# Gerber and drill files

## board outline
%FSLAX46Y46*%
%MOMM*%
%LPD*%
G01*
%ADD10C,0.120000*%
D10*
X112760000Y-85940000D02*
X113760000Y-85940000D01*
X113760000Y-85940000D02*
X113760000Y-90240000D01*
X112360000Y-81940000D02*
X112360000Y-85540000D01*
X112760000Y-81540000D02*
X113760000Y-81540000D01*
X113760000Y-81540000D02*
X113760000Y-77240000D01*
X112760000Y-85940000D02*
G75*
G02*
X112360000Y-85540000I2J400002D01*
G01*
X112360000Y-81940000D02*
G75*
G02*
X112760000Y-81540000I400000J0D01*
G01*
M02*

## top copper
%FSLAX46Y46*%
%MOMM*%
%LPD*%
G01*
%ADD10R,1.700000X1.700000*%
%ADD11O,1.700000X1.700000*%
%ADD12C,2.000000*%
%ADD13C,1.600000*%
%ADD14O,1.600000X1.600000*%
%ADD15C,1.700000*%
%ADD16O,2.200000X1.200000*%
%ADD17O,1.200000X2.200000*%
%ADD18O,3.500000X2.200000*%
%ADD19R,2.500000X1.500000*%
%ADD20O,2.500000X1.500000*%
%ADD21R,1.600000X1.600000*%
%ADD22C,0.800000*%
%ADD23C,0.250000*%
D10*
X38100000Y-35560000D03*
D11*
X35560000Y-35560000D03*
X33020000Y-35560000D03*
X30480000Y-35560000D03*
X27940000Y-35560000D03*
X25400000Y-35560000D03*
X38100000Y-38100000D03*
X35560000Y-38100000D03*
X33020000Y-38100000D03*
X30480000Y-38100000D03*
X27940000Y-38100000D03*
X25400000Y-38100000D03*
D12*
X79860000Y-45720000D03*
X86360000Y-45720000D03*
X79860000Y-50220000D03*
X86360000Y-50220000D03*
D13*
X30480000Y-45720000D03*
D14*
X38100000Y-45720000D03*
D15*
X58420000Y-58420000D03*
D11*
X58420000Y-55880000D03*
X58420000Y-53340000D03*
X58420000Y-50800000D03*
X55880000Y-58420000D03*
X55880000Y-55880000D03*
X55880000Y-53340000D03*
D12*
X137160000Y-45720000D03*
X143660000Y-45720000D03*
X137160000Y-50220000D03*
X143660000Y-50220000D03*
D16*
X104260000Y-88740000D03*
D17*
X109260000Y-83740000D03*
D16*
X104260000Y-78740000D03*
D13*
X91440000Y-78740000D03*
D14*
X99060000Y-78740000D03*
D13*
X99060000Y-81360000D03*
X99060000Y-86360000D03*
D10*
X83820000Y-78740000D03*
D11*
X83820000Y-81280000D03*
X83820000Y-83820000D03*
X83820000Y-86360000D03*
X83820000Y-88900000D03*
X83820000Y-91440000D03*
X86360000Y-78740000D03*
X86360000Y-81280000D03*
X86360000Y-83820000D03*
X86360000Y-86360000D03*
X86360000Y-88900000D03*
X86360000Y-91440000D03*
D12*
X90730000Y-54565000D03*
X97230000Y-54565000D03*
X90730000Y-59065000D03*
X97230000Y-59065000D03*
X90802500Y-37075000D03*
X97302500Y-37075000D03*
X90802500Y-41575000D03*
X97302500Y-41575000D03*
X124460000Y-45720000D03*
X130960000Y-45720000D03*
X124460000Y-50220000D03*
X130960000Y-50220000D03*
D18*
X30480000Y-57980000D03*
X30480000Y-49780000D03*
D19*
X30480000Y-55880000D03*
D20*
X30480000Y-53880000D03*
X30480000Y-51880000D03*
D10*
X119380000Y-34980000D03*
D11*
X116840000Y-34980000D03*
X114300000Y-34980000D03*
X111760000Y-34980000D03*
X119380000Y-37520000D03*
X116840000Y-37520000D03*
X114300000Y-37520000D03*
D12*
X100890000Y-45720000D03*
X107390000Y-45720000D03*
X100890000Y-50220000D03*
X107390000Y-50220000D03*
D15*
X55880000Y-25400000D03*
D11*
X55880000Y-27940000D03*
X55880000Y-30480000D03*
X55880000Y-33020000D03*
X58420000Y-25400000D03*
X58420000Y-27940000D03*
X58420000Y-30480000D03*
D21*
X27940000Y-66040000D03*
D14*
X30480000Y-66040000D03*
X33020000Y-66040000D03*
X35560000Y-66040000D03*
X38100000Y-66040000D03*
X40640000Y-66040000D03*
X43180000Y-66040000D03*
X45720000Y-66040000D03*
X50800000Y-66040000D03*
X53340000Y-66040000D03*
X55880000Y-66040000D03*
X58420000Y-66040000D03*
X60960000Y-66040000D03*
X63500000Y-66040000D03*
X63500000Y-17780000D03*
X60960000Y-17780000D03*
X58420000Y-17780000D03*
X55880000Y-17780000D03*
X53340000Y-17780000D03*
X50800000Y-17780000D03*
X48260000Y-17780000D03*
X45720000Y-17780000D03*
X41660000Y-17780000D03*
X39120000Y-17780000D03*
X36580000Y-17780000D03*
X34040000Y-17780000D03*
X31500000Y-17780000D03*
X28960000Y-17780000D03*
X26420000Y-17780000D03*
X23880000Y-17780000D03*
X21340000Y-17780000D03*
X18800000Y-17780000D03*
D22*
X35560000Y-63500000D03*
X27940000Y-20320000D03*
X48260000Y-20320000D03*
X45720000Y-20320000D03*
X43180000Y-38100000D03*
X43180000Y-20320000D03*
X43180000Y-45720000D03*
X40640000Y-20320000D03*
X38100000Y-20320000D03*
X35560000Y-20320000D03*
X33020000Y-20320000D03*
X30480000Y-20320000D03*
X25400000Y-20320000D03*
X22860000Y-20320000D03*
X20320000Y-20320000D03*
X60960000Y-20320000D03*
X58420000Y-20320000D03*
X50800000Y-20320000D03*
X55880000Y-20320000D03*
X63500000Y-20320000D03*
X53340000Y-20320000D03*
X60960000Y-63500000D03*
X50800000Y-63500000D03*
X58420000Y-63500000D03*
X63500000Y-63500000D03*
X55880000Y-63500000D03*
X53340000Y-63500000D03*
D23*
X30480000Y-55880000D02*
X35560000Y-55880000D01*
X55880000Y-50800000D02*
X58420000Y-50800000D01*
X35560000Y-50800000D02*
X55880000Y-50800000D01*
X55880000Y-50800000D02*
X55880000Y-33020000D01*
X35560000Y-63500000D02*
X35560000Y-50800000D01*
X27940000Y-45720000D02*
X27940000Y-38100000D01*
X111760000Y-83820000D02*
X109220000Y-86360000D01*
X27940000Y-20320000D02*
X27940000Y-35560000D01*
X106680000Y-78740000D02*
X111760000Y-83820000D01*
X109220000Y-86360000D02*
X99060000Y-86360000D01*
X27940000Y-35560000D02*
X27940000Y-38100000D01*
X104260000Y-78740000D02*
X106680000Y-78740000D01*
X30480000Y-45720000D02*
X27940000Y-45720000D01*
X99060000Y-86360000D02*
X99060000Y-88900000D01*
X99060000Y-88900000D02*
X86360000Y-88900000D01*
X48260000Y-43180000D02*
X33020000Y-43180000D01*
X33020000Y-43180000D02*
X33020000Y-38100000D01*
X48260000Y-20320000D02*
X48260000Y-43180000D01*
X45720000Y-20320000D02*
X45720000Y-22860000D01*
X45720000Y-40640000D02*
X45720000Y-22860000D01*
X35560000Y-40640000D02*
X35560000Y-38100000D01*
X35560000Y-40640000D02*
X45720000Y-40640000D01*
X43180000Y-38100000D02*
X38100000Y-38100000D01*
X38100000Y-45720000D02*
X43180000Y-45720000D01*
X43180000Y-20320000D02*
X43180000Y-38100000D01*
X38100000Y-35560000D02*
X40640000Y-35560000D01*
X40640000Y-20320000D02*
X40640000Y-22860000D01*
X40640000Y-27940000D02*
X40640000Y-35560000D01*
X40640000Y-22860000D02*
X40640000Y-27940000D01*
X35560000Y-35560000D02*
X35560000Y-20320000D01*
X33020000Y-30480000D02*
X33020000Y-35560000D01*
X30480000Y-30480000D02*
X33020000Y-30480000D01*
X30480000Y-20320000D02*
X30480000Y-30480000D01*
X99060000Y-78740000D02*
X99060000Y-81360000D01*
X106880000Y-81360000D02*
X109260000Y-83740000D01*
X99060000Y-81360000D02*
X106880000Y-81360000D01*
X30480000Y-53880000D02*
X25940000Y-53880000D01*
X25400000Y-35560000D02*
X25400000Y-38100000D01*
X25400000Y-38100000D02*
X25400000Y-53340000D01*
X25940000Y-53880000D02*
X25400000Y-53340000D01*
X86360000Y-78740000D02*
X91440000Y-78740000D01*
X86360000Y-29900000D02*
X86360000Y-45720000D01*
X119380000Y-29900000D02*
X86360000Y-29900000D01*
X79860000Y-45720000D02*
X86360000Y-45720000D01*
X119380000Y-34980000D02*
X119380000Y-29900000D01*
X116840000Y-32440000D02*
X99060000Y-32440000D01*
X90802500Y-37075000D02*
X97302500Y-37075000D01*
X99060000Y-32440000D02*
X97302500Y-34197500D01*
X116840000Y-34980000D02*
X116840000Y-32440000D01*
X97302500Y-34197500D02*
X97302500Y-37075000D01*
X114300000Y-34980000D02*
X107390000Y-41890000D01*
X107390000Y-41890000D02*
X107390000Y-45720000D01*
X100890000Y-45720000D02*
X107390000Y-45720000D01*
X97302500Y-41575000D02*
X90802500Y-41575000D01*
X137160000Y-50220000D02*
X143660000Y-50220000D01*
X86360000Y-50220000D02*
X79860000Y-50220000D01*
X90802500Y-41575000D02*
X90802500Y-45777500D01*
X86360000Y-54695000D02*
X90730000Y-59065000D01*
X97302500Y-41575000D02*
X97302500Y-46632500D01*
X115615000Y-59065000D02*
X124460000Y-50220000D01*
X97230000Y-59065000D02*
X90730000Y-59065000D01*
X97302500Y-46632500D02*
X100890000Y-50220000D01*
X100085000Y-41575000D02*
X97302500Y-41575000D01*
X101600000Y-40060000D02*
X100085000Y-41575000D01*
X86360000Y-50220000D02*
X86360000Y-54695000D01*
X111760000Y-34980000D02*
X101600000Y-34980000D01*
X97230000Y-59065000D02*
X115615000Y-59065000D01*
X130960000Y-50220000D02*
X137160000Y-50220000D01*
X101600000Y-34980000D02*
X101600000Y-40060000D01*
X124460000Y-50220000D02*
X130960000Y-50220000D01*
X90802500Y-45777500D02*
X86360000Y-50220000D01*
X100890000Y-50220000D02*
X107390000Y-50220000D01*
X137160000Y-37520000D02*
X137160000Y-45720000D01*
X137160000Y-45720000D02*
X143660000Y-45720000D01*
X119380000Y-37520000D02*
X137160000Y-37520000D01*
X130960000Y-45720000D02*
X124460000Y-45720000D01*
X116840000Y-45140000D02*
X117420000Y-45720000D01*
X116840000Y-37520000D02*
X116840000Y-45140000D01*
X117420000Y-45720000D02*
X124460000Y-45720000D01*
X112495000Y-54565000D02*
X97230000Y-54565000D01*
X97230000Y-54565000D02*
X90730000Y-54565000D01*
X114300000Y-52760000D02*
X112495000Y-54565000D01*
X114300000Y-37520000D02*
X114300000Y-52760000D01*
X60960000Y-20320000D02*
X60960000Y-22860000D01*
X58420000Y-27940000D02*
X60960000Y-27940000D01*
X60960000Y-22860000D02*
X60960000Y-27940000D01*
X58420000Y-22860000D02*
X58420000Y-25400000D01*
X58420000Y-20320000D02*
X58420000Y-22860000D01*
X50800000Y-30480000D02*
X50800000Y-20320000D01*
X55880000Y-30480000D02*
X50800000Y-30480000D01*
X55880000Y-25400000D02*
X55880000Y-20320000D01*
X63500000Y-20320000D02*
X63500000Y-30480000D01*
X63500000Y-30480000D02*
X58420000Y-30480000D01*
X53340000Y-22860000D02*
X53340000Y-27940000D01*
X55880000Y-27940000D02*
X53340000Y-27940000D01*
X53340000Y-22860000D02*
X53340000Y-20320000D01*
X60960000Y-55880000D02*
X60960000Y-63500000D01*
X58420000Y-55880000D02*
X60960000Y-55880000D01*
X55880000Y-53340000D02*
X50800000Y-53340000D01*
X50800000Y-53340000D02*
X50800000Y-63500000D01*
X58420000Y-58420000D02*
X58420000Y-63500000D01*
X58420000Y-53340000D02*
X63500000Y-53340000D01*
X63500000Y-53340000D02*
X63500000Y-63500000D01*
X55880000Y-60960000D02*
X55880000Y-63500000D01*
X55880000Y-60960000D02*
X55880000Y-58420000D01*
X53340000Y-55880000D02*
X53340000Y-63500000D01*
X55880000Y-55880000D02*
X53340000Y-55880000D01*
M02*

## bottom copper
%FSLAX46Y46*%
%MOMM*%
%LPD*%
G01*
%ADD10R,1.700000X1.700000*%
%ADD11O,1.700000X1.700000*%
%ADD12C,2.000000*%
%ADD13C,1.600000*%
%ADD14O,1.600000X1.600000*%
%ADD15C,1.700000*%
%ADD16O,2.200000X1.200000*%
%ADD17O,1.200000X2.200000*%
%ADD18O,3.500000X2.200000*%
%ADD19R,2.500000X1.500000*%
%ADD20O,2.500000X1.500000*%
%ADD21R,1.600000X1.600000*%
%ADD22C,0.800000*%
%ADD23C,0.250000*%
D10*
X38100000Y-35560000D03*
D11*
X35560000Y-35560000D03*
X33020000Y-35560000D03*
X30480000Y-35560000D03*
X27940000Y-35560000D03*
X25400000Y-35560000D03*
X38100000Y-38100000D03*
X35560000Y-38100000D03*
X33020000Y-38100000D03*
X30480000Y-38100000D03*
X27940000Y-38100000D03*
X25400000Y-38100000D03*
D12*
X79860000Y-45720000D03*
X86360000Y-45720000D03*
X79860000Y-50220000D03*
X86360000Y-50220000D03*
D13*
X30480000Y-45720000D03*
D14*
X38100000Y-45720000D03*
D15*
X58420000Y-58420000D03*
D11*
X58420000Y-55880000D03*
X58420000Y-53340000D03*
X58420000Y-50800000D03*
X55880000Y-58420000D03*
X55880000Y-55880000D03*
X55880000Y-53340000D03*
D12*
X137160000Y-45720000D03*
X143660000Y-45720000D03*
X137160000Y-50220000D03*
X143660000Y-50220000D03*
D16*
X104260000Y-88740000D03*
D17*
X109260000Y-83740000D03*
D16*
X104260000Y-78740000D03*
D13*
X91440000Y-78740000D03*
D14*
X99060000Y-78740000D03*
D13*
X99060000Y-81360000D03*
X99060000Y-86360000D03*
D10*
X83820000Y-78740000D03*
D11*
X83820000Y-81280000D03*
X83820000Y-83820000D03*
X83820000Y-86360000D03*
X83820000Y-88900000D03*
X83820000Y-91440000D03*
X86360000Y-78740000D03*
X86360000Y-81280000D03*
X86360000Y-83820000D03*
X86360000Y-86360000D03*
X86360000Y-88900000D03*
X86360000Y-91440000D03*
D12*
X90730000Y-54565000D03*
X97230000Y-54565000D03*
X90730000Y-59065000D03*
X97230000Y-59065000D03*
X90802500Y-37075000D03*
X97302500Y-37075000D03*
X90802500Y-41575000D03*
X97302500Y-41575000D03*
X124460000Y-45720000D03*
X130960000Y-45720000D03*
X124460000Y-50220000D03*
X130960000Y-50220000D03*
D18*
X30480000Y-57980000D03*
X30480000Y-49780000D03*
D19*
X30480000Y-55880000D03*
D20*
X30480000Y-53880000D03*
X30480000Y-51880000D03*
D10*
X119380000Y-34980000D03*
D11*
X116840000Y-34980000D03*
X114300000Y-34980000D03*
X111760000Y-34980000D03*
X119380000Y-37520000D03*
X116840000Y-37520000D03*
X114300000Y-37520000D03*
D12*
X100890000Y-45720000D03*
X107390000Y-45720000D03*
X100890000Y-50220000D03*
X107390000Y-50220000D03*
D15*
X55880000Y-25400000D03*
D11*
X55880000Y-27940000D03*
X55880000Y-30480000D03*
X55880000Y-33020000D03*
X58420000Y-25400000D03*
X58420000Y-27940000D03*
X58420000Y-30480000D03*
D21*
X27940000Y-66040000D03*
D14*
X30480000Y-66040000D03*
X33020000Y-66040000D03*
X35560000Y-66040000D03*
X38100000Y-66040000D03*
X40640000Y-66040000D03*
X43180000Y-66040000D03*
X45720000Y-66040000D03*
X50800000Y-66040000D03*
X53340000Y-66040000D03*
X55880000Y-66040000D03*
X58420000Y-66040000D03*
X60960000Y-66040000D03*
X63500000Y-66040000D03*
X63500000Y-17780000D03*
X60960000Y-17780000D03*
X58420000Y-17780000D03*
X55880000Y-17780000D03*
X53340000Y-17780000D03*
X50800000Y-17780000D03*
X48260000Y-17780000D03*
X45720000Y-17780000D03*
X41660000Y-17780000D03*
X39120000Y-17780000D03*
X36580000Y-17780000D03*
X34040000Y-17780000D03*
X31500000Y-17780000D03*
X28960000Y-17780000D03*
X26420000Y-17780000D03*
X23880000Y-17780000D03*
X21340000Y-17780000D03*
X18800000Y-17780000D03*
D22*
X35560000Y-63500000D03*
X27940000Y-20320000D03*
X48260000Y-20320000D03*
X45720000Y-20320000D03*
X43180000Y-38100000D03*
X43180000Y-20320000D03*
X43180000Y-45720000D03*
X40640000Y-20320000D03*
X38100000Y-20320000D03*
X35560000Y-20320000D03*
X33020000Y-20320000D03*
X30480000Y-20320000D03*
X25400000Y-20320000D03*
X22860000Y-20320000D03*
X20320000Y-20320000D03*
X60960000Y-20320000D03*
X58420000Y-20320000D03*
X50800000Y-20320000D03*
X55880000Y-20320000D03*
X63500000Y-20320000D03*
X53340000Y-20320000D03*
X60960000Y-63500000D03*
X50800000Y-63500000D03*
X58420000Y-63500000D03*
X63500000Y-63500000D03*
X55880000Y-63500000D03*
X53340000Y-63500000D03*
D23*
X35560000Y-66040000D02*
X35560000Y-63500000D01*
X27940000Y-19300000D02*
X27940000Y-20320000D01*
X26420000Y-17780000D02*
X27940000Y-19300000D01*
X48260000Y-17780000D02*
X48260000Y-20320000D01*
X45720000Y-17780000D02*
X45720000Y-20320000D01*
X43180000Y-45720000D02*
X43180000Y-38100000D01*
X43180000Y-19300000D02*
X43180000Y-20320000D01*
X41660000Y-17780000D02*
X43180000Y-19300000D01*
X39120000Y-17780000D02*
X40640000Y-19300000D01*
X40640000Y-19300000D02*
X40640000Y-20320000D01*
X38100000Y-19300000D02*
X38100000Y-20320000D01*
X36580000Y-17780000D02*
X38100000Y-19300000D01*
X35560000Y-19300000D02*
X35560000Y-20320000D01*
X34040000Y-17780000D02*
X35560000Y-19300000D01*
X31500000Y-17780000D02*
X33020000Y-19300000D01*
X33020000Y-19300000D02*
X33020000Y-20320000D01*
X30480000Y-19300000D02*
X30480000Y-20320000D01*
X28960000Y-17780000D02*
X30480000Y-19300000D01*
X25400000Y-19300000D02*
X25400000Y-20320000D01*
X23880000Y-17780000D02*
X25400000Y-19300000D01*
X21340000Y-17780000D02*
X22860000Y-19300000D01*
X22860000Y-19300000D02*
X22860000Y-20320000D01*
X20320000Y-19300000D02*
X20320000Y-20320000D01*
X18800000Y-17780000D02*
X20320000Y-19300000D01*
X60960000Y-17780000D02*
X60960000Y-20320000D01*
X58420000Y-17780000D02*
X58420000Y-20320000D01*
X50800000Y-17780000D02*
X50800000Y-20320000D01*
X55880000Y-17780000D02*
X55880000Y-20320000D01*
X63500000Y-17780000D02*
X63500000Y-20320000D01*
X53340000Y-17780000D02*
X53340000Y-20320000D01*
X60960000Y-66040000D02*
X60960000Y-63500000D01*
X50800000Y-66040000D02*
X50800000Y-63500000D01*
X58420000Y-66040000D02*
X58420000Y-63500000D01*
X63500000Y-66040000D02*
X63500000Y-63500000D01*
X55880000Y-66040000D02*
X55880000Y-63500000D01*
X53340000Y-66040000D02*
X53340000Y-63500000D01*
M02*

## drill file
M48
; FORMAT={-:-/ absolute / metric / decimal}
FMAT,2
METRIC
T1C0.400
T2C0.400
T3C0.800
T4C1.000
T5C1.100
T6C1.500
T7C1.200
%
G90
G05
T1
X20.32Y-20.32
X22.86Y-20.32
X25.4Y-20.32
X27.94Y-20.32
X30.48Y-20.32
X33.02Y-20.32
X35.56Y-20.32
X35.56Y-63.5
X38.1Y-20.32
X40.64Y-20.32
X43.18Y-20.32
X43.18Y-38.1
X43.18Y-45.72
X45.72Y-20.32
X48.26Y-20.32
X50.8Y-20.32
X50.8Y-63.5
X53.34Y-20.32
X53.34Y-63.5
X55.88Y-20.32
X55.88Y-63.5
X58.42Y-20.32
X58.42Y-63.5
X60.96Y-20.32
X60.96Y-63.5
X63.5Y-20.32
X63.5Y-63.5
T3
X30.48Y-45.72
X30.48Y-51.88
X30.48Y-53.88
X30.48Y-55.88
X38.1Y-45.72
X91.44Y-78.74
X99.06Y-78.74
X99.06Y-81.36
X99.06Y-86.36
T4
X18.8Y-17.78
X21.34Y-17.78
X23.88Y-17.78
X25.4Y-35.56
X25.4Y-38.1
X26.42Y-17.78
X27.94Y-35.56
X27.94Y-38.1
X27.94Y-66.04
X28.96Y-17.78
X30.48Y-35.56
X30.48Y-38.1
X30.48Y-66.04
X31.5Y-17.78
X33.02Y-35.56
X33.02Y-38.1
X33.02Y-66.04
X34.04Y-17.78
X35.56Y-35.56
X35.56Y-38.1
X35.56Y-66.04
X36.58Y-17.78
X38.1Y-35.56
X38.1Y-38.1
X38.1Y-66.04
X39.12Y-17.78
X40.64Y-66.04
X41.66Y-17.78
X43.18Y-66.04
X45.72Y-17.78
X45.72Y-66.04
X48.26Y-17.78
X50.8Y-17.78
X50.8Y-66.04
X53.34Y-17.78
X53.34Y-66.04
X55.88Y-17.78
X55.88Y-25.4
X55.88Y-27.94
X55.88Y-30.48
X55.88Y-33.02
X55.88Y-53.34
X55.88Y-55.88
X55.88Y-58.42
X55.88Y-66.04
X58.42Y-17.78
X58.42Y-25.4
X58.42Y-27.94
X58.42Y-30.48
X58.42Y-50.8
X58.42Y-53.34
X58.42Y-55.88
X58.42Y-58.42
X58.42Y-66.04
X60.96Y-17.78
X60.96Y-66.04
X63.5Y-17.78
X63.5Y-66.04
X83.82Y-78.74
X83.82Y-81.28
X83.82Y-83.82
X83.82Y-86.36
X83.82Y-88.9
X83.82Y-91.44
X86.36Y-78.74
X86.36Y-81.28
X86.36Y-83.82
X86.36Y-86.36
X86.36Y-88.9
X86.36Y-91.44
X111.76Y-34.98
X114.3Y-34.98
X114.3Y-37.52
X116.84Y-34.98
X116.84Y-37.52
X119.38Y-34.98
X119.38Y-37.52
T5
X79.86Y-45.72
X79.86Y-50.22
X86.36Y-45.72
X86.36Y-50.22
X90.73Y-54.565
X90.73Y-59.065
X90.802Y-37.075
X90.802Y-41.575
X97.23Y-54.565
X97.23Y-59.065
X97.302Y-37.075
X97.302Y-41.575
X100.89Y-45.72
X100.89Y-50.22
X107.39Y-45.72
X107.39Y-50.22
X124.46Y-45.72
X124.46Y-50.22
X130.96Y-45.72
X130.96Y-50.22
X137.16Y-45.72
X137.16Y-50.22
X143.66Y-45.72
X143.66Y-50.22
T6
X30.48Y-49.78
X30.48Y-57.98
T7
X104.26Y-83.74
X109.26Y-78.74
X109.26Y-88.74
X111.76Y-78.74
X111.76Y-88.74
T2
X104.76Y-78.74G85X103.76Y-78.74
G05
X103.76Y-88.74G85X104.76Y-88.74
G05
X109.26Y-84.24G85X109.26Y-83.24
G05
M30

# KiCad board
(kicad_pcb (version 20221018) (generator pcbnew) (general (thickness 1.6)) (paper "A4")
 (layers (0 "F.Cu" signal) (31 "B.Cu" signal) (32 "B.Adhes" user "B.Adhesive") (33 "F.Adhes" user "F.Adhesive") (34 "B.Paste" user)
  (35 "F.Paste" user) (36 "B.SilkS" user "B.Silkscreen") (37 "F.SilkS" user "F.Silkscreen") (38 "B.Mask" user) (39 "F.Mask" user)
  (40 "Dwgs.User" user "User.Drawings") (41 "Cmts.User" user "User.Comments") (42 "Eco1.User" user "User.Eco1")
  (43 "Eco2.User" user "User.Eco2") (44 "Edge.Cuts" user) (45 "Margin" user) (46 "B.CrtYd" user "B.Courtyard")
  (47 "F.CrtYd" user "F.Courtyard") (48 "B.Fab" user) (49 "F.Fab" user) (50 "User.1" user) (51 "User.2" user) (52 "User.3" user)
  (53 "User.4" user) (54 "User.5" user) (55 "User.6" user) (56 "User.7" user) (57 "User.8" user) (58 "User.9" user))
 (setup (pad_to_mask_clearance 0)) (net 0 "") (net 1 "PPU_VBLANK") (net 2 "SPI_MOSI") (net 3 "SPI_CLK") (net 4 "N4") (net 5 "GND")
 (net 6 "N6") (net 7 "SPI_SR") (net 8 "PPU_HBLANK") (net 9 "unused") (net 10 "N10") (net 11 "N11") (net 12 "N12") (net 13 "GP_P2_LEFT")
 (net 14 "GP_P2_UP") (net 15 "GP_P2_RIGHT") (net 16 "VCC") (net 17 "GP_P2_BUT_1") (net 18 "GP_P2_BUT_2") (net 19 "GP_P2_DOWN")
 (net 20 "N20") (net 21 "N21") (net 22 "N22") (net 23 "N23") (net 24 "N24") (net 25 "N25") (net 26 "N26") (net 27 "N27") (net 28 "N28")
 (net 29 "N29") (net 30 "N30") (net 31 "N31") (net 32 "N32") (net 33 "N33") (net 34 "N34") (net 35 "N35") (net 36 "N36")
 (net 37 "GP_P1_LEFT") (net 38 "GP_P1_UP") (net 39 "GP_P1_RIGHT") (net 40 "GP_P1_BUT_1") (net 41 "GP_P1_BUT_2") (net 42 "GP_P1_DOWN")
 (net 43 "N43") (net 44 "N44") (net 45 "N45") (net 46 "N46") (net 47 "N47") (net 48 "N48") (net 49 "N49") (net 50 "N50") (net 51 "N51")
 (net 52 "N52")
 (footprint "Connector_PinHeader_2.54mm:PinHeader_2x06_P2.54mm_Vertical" (layer "F.Cu") (at 38.1 35.56 -90)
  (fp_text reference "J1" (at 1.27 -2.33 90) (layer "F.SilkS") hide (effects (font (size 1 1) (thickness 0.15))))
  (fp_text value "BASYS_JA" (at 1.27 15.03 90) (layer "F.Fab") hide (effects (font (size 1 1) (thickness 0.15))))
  (pad "1" thru_hole rect (at 0 0 270) (size 1.7 1.7) (drill 1) (layers "*.Cu" "*.Mask") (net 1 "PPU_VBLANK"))
  (pad "2" thru_hole oval (at 0 2.54 270) (size 1.7 1.7) (drill 1) (layers "*.Cu" "*.Mask") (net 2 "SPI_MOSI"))
  (pad "3" thru_hole oval (at 0 5.08 270) (size 1.7 1.7) (drill 1) (layers "*.Cu" "*.Mask") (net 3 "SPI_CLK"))
  (pad "4" thru_hole oval (at 0 7.62 270) (size 1.7 1.7) (drill 1) (layers "*.Cu" "*.Mask") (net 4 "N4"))
  (pad "5" thru_hole oval (at 0 10.16 270) (size 1.7 1.7) (drill 1) (layers "*.Cu" "*.Mask") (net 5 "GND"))
  (pad "6" thru_hole oval (at 0 12.7 270) (size 1.7 1.7) (drill 1) (layers "*.Cu" "*.Mask") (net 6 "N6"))
  (pad "7" thru_hole oval (at 2.54 0 270) (size 1.7 1.7) (drill 1) (layers "*.Cu" "*.Mask") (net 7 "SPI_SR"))
  (pad "8" thru_hole oval (at 2.54 2.54 270) (size 1.7 1.7) (drill 1) (layers "*.Cu" "*.Mask") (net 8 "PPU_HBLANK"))
  (pad "9" thru_hole oval (at 2.54 5.08 270) (size 1.7 1.7) (drill 1) (layers "*.Cu" "*.Mask") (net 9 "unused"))
  (pad "10" thru_hole oval (at 2.54 7.62 270) (size 1.7 1.7) (drill 1) (layers "*.Cu" "*.Mask") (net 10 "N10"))
  (pad "11" thru_hole oval (at 2.54 10.16 270) (size 1.7 1.7) (drill 1) (layers "*.Cu" "*.Mask") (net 5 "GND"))
  (pad "12" thru_hole oval (at 2.54 12.7 270) (size 1.7 1.7) (drill 1) (layers "*.Cu" "*.Mask") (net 6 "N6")))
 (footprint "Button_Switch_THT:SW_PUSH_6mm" (layer "F.Cu") (at 79.86 45.72)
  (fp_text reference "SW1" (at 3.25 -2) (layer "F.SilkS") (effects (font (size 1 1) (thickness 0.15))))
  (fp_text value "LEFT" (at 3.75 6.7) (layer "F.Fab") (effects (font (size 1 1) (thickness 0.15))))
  (pad "1" thru_hole circle (at 0 0 90) (size 2 2) (drill 1.1) (layers "*.Cu" "*.Mask") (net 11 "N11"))
  (pad "1" thru_hole circle (at 6.5 0 90) (size 2 2) (drill 1.1) (layers "*.Cu" "*.Mask") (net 11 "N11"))
  (pad "2" thru_hole circle (at 0 4.5 90) (size 2 2) (drill 1.1) (layers "*.Cu" "*.Mask") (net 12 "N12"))
  (pad "2" thru_hole circle (at 6.5 4.5 90) (size 2 2) (drill 1.1) (layers "*.Cu" "*.Mask") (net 12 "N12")))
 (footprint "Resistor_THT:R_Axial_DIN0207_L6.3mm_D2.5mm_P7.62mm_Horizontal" (layer "F.Cu") (at 30.48 45.72)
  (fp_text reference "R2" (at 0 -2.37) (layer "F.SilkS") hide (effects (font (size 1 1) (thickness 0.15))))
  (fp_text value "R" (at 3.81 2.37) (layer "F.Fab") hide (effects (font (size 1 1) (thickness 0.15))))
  (pad "1" thru_hole circle (at 0 0) (size 1.6 1.6) (drill 0.8) (layers "*.Cu" "*.Mask") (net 5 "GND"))
  (pad "2" thru_hole oval (at 7.62 0) (size 1.6 1.6) (drill 0.8) (layers "*.Cu" "*.Mask") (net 7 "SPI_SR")))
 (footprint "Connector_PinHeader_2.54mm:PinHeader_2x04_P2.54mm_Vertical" (layer "F.Cu") (at 58.42 58.42 180)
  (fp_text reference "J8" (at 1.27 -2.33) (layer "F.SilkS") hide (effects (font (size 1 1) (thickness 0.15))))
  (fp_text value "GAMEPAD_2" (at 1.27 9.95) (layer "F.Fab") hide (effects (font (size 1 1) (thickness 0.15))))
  (pad "1" thru_hole circle (at 0 0 180) (size 1.7 1.7) (drill 1) (layers "*.Cu" "*.Mask") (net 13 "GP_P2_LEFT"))
  (pad "2" thru_hole oval (at 0 2.54 180) (size 1.7 1.7) (drill 1) (layers "*.Cu" "*.Mask") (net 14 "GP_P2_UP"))
  (pad "3" thru_hole oval (at 0 5.08 180) (size 1.7 1.7) (drill 1) (layers "*.Cu" "*.Mask") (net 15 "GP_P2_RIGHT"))
  (pad "4" thru_hole oval (at 0 7.62 180) (size 1.7 1.7) (drill 1) (layers "*.Cu" "*.Mask") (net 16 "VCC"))
  (pad "5" thru_hole oval (at 2.54 0 180) (size 1.7 1.7) (drill 1) (layers "*.Cu" "*.Mask") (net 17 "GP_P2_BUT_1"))
  (pad "6" thru_hole oval (at 2.54 2.54 180) (size 1.7 1.7) (drill 1) (layers "*.Cu" "*.Mask") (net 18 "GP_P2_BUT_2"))
  (pad "7" thru_hole oval (at 2.54 5.08 180) (size 1.7 1.7) (drill 1) (layers "*.Cu" "*.Mask") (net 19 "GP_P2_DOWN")))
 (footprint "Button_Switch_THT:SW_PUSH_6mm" (layer "F.Cu") (at 137.16 45.72)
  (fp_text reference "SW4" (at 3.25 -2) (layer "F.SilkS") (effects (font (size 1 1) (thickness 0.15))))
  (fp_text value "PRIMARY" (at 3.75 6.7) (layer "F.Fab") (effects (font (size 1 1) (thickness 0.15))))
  (pad "1" thru_hole circle (at 0 0 90) (size 2 2) (drill 1.1) (layers "*.Cu" "*.Mask") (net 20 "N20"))
  (pad "1" thru_hole circle (at 6.5 0 90) (size 2 2) (drill 1.1) (layers "*.Cu" "*.Mask") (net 20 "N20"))
  (pad "2" thru_hole circle (at 0 4.5 90) (size 2 2) (drill 1.1) (layers "*.Cu" "*.Mask") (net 12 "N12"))
  (pad "2" thru_hole circle (at 6.5 4.5 90) (size 2 2) (drill 1.1) (layers "*.Cu" "*.Mask") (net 12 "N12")))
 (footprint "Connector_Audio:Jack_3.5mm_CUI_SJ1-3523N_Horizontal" (layer "F.Cu") (at 109.26 83.74 90)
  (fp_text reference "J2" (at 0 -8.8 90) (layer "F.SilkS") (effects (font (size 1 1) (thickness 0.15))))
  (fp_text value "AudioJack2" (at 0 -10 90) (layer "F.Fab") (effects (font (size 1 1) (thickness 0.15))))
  (fp_line (start -2.2 3.5) (end -2.2 4.5) (stroke (width 0.12) (type solid)) (layer "Edge.Cuts"))
  (fp_line (start -2.2 4.5) (end -6.5 4.5) (stroke (width 0.12) (type solid)) (layer "Edge.Cuts"))
  (fp_line (start 1.8 3.1) (end -1.8 3.1) (stroke (width 0.12) (type solid)) (layer "Edge.Cuts"))
  (fp_line (start 2.2 3.5) (end 2.2 4.5) (stroke (width 0.12) (type solid)) (layer "Edge.Cuts"))
  (fp_line (start 2.2 4.5) (end 6.5 4.5) (stroke (width 0.12) (type solid)) (layer "Edge.Cuts"))
  (fp_arc (start -2.2 3.5) (mid -2.082842 3.217158) (end -1.8 3.1) (stroke (width 0.12) (type solid)) (layer "Edge.Cuts"))
  (fp_arc (start 1.8 3.1) (mid 2.082843 3.217157) (end 2.2 3.5) (stroke (width 0.12) (type solid)) (layer "Edge.Cuts"))
  (pad "" np_thru_hole circle (at -5 0 90) (size 1.2 1.2) (drill 1.2) (layers "*.Cu"))
  (pad "" np_thru_hole circle (at -5 2.5 90) (size 1.2 1.2) (drill 1.2) (layers "*.Cu"))
  (pad "" np_thru_hole circle (at 0 -5 90) (size 1.2 1.2) (drill 1.2) (layers "*.Cu"))
  (pad "" np_thru_hole circle (at 5 0 90) (size 1.2 1.2) (drill 1.2) (layers "*.Cu"))
  (pad "" np_thru_hole circle (at 5 2.5 90) (size 1.2 1.2) (drill 1.2) (layers "*.Cu"))
  (pad "R" thru_hole oval (at -5 -5 90) (size 1.2 2.2) (drill oval 0.4 1.4) (layers "*.Cu" "*.Mask"))
  (pad "S" thru_hole oval (at 0 0 90) (size 2.2 1.2) (drill oval 1.4 0.4) (layers "*.Cu" "*.Mask") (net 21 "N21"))
  (pad "T" thru_hole oval (at 5 -5 270) (size 1.2 2.2) (drill oval 0.4 1.4) (layers "*.Cu" "*.Mask") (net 5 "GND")))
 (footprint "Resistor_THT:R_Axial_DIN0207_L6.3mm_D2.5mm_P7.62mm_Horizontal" (layer "F.Cu") (at 91.44 78.74)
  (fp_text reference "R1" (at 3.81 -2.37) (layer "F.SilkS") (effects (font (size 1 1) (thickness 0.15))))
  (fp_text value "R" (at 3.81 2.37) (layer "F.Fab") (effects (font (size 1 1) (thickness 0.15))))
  (pad "1" thru_hole circle (at 0 0) (size 1.6 1.6) (drill 0.8) (layers "*.Cu" "*.Mask") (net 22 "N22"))
  (pad "2" thru_hole oval (at 7.62 0) (size 1.6 1.6) (drill 0.8) (layers "*.Cu" "*.Mask") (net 21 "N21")))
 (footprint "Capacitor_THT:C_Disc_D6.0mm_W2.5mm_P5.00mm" (layer "F.Cu") (at 99.06 81.36 -90)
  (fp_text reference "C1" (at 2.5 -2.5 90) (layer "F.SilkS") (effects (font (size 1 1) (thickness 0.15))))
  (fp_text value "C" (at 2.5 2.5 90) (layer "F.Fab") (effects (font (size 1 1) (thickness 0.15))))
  (pad "1" thru_hole circle (at 0 0 270) (size 1.6 1.6) (drill 0.8) (layers "*.Cu" "*.Mask") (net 21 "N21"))
  (pad "2" thru_hole circle (at 5 0 270) (size 1.6 1.6) (drill 0.8) (layers "*.Cu" "*.Mask") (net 5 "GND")))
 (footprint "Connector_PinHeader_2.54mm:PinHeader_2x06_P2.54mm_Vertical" (layer "F.Cu") (at 83.82 78.74)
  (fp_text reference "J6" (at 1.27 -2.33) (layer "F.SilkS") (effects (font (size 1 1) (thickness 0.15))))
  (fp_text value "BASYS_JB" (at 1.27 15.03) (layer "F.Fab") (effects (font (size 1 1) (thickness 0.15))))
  (pad "1" thru_hole rect (at 0 0) (size 1.7 1.7) (drill 1) (layers "*.Cu" "*.Mask") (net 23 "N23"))
  (pad "2" thru_hole oval (at 0 2.54) (size 1.7 1.7) (drill 1) (layers "*.Cu" "*.Mask") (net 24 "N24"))
  (pad "3" thru_hole oval (at 0 5.08) (size 1.7 1.7) (drill 1) (layers "*.Cu" "*.Mask") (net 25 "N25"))
  (pad "4" thru_hole oval (at 0 7.62) (size 1.7 1.7) (drill 1) (layers "*.Cu" "*.Mask") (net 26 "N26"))
  (pad "5" thru_hole oval (at 0 10.16) (size 1.7 1.7) (drill 1) (layers "*.Cu" "*.Mask") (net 5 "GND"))
  (pad "6" thru_hole oval (at 0 12.7) (size 1.7 1.7) (drill 1) (layers "*.Cu" "*.Mask") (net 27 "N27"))
  (pad "7" thru_hole oval (at 2.54 0) (size 1.7 1.7) (drill 1) (layers "*.Cu" "*.Mask") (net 22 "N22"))
  (pad "8" thru_hole oval (at 2.54 2.54) (size 1.7 1.7) (drill 1) (layers "*.Cu" "*.Mask") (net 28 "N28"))
  (pad "9" thru_hole oval (at 2.54 5.08) (size 1.7 1.7) (drill 1) (layers "*.Cu" "*.Mask") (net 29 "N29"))
  (pad "10" thru_hole oval (at 2.54 7.62) (size 1.7 1.7) (drill 1) (layers "*.Cu" "*.Mask") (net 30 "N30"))
  (pad "11" thru_hole oval (at 2.54 10.16) (size 1.7 1.7) (drill 1) (layers "*.Cu" "*.Mask") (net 5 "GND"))
  (pad "12" thru_hole oval (at 2.54 12.7) (size 1.7 1.7) (drill 1) (layers "*.Cu" "*.Mask") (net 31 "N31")))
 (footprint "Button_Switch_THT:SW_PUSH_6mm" (layer "F.Cu") (at 90.73 54.565)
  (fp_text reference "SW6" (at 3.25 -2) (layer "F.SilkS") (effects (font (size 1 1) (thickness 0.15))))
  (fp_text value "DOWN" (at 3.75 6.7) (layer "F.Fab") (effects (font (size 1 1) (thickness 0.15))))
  (pad "1" thru_hole circle (at 0 0 90) (size 2 2) (drill 1.1) (layers "*.Cu" "*.Mask") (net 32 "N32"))
  (pad "1" thru_hole circle (at 6.5 0 90) (size 2 2) (drill 1.1) (layers "*.Cu" "*.Mask") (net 32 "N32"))
  (pad "2" thru_hole circle (at 0 4.5 90) (size 2 2) (drill 1.1) (layers "*.Cu" "*.Mask") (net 12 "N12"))
  (pad "2" thru_hole circle (at 6.5 4.5 90) (size 2 2) (drill 1.1) (layers "*.Cu" "*.Mask") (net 12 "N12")))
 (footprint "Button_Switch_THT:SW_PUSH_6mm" (layer "F.Cu") (at 90.8025 37.075)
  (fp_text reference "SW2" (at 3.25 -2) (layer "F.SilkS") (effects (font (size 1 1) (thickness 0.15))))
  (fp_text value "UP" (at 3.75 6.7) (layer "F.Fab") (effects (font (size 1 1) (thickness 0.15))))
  (pad "1" thru_hole circle (at 0 0 90) (size 2 2) (drill 1.1) (layers "*.Cu" "*.Mask") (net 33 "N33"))
  (pad "1" thru_hole circle (at 6.5 0 90) (size 2 2) (drill 1.1) (layers "*.Cu" "*.Mask") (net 33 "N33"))
  (pad "2" thru_hole circle (at 0 4.5 90) (size 2 2) (drill 1.1) (layers "*.Cu" "*.Mask") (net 12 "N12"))
  (pad "2" thru_hole circle (at 6.5 4.5 90) (size 2 2) (drill 1.1) (layers "*.Cu" "*.Mask") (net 12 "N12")))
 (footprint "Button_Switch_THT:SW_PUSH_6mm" (layer "F.Cu") (at 124.46 45.72)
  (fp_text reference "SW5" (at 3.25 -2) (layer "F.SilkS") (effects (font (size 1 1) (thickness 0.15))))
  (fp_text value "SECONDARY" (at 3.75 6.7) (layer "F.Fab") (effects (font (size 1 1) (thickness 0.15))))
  (pad "1" thru_hole circle (at 0 0 90) (size 2 2) (drill 1.1) (layers "*.Cu" "*.Mask") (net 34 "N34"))
  (pad "1" thru_hole circle (at 6.5 0 90) (size 2 2) (drill 1.1) (layers "*.Cu" "*.Mask") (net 34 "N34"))
  (pad "2" thru_hole circle (at 0 4.5 90) (size 2 2) (drill 1.1) (layers "*.Cu" "*.Mask") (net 12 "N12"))
  (pad "2" thru_hole circle (at 6.5 4.5 90) (size 2 2) (drill 1.1) (layers "*.Cu" "*.Mask") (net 12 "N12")))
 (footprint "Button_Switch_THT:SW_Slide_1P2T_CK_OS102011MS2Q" (layer "F.Cu") (at 30.48 55.88 90)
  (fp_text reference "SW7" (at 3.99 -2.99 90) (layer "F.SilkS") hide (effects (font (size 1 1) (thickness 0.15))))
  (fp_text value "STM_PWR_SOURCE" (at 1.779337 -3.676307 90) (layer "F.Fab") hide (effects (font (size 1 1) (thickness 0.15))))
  (pad "" thru_hole oval (at -2.1 0 90) (size 2.2 3.5) (drill 1.5) (layers "*.Cu" "*.Mask"))
  (pad "" thru_hole oval (at 6.1 0 90) (size 2.2 3.5) (drill 1.5) (layers "*.Cu" "*.Mask"))
  (pad "1" thru_hole rect (at 0 0 90) (size 1.5 2.5) (drill 0.8) (layers "*.Cu" "*.Mask") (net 16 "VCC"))
  (pad "2" thru_hole oval (at 2 0 90) (size 1.5 2.5) (drill 0.8) (layers "*.Cu" "*.Mask") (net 6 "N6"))
  (pad "3" thru_hole oval (at 4 0 90) (size 1.5 2.5) (drill 0.8) (layers "*.Cu" "*.Mask") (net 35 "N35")))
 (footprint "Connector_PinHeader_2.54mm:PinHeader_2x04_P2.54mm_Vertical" (layer "F.Cu") (at 119.38 34.98 -90)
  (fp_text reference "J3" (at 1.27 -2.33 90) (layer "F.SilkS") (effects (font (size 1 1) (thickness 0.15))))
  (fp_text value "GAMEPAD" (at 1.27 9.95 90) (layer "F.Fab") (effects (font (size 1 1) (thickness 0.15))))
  (pad "1" thru_hole rect (at 0 0 270) (size 1.7 1.7) (drill 1) (layers "*.Cu" "*.Mask") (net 11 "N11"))
  (pad "2" thru_hole oval (at 0 2.54 270) (size 1.7 1.7) (drill 1) (layers "*.Cu" "*.Mask") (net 33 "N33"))
  (pad "3" thru_hole oval (at 0 5.08 270) (size 1.7 1.7) (drill 1) (layers "*.Cu" "*.Mask") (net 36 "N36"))
  (pad "4" thru_hole oval (at 0 7.62 270) (size 1.7 1.7) (drill 1) (layers "*.Cu" "*.Mask") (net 12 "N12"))
  (pad "5" thru_hole oval (at 2.54 0 270) (size 1.7 1.7) (drill 1) (layers "*.Cu" "*.Mask" "B.SilkS") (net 20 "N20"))
  (pad "6" thru_hole oval (at 2.54 2.54 270) (size 1.7 1.7) (drill 1) (layers "*.Cu" "*.Mask") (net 34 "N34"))
  (pad "7" thru_hole oval (at 2.54 5.08 270) (size 1.7 1.7) (drill 1) (layers "*.Cu" "*.Mask") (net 32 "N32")))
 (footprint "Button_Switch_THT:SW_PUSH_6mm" (layer "F.Cu") (at 100.89 45.72)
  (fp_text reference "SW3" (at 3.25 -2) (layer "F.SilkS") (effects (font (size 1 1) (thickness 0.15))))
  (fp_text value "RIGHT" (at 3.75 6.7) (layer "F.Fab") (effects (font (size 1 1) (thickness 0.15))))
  (pad "1" thru_hole circle (at 0 0 90) (size 2 2) (drill 1.1) (layers "*.Cu" "*.Mask") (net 36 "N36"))
  (pad "1" thru_hole circle (at 6.5 0 90) (size 2 2) (drill 1.1) (layers "*.Cu" "*.Mask") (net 36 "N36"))
  (pad "2" thru_hole circle (at 0 4.5 90) (size 2 2) (drill 1.1) (layers "*.Cu" "*.Mask") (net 12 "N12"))
  (pad "2" thru_hole circle (at 6.5 4.5 90) (size 2 2) (drill 1.1) (layers "*.Cu" "*.Mask") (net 12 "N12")))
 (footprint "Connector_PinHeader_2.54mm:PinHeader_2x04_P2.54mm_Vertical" (layer "F.Cu") (at 55.88 25.4)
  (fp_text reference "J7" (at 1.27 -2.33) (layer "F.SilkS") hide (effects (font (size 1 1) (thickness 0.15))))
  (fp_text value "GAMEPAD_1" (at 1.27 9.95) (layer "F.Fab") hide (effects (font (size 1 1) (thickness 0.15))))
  (pad "1" thru_hole circle (at 0 0) (size 1.7 1.7) (drill 1) (layers "*.Cu" "*.Mask") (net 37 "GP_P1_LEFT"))
  (pad "2" thru_hole oval (at 0 2.54) (size 1.7 1.7) (drill 1) (layers "*.Cu" "*.Mask") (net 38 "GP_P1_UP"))
  (pad "3" thru_hole oval (at 0 5.08) (size 1.7 1.7) (drill 1) (layers "*.Cu" "*.Mask") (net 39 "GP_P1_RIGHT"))
  (pad "4" thru_hole oval (at 0 7.62) (size 1.7 1.7) (drill 1) (layers "*.Cu" "*.Mask") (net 16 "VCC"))
  (pad "5" thru_hole oval (at 2.54 0) (size 1.7 1.7) (drill 1) (layers "*.Cu" "*.Mask") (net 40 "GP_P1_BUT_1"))
  (pad "6" thru_hole oval (at 2.54 2.54) (size 1.7 1.7) (drill 1) (layers "*.Cu" "*.Mask") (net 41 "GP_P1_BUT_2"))
  (pad "7" thru_hole oval (at 2.54 5.08) (size 1.7 1.7) (drill 1) (layers "*.Cu" "*.Mask") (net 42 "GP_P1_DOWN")))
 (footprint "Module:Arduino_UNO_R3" (layer "B.Cu") (at 27.94 66.04)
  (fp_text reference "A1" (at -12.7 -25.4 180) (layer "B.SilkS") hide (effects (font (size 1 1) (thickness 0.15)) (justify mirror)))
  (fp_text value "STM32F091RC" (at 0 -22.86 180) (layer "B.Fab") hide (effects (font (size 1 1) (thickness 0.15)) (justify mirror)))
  (pad "1" thru_hole rect (at 0 0 270) (size 1.6 1.6) (drill 1) (layers "*.Cu" "*.Mask") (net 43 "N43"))
  (pad "2" thru_hole oval (at 2.54 0 270) (size 1.6 1.6) (drill 1) (layers "*.Cu" "*.Mask") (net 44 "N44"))
  (pad "3" thru_hole oval (at 5.08 0 270) (size 1.6 1.6) (drill 1) (layers "*.Cu" "*.Mask") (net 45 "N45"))
  (pad "4" thru_hole oval (at 7.62 0 270) (size 1.6 1.6) (drill 1) (layers "*.Cu" "*.Mask") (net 16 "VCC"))
  (pad "5" thru_hole oval (at 10.16 0 270) (size 1.6 1.6) (drill 1) (layers "*.Cu" "*.Mask") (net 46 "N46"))
  (pad "6" thru_hole oval (at 12.7 0 270) (size 1.6 1.6) (drill 1) (layers "*.Cu" "*.Mask") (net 5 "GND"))
  (pad "7" thru_hole oval (at 15.24 0 270) (size 1.6 1.6) (drill 1) (layers "*.Cu" "*.Mask") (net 5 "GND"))
  (pad "8" thru_hole oval (at 17.78 0 270) (size 1.6 1.6) (drill 1) (layers "*.Cu" "*.Mask") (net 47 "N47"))
  (pad "9" thru_hole oval (at 22.86 0 270) (size 1.6 1.6) (drill 1) (layers "*.Cu" "*.Mask") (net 19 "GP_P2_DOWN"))
  (pad "10" thru_hole oval (at 25.4 0 270) (size 1.6 1.6) (drill 1) (layers "*.Cu" "*.Mask") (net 18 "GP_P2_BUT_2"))
  (pad "11" thru_hole oval (at 27.94 0 270) (size 1.6 1.6) (drill 1) (layers "*.Cu" "*.Mask") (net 17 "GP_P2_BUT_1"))
  (pad "12" thru_hole oval (at 30.48 0 270) (size 1.6 1.6) (drill 1) (layers "*.Cu" "*.Mask") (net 13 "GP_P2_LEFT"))
  (pad "13" thru_hole oval (at 33.02 0 270) (size 1.6 1.6) (drill 1) (layers "*.Cu" "*.Mask") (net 14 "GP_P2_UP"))
  (pad "14" thru_hole oval (at 35.56 0 270) (size 1.6 1.6) (drill 1) (layers "*.Cu" "*.Mask") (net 15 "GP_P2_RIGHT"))
  (pad "15" thru_hole oval (at 35.56 -48.26 270) (size 1.6 1.6) (drill 1) (layers "*.Cu" "*.Mask") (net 42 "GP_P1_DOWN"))
  (pad "16" thru_hole oval (at 33.02 -48.26 270) (size 1.6 1.6) (drill 1) (layers "*.Cu" "*.Mask") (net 41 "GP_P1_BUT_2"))
  (pad "17" thru_hole oval (at 30.48 -48.26 270) (size 1.6 1.6) (drill 1) (layers "*.Cu" "*.Mask") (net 40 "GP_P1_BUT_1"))
  (pad "18" thru_hole oval (at 27.94 -48.26 270) (size 1.6 1.6) (drill 1) (layers "*.Cu" "*.Mask") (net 37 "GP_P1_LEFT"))
  (pad "19" thru_hole oval (at 25.4 -48.26 270) (size 1.6 1.6) (drill 1) (layers "*.Cu" "*.Mask") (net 38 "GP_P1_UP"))
  (pad "20" thru_hole oval (at 22.86 -48.26 270) (size 1.6 1.6) (drill 1) (layers "*.Cu" "*.Mask") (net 39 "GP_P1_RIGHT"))
  (pad "21" thru_hole oval (at 20.32 -48.26 270) (size 1.6 1.6) (drill 1) (layers "*.Cu" "*.Mask") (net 9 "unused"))
  (pad "22" thru_hole oval (at 17.78 -48.26 270) (size 1.6 1.6) (drill 1) (layers "*.Cu" "*.Mask") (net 8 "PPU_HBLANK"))
  (pad "23" thru_hole oval (at 13.72 -48.26 270) (size 1.6 1.6) (drill 1) (layers "*.Cu" "*.Mask") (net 7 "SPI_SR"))
  (pad "24" thru_hole oval (at 11.18 -48.26 270) (size 1.6 1.6) (drill 1) (layers "*.Cu" "*.Mask") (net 1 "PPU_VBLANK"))
  (pad "25" thru_hole oval (at 8.64 -48.26 270) (size 1.6 1.6) (drill 1) (layers "*.Cu" "*.Mask") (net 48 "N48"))
  (pad "26" thru_hole oval (at 6.1 -48.26 270) (size 1.6 1.6) (drill 1) (layers "*.Cu" "*.Mask") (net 2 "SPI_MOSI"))
  (pad "27" thru_hole oval (at 3.56 -48.26 270) (size 1.6 1.6) (drill 1) (layers "*.Cu" "*.Mask") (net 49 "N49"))
  (pad "28" thru_hole oval (at 1.02 -48.26 270) (size 1.6 1.6) (drill 1) (layers "*.Cu" "*.Mask") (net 3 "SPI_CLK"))
  (pad "29" thru_hole oval (at -1.52 -48.26 270) (size 1.6 1.6) (drill 1) (layers "*.Cu" "*.Mask") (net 5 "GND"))
  (pad "30" thru_hole oval (at -4.06 -48.26 270) (size 1.6 1.6) (drill 1) (layers "*.Cu" "*.Mask") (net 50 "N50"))
  (pad "31" thru_hole oval (at -6.6 -48.26 270) (size 1.6 1.6) (drill 1) (layers "*.Cu" "*.Mask") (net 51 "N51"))
  (pad "32" thru_hole oval (at -9.14 -48.26 270) (size 1.6 1.6) (drill 1) (layers "*.Cu" "*.Mask") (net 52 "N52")))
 (segment (start 30.48 55.88) (end 35.56 55.88) (width 0.25) (layer "F.Cu") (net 16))
 (segment (start 55.88 50.8) (end 58.42 50.8) (width 0.25) (layer "F.Cu") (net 16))
 (segment (start 35.56 50.8) (end 55.88 50.8) (width 0.25) (layer "F.Cu") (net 16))
 (segment (start 55.88 50.8) (end 55.88 33.02) (width 0.25) (layer "F.Cu") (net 16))
 (segment (start 35.56 63.5) (end 35.56 50.8) (width 0.25) (layer "F.Cu") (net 16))
 (via (at 35.56 63.5) (size 0.8) (drill 0.4) (layers "F.Cu" "B.Cu") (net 16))
 (segment (start 35.56 66.04) (end 35.56 63.5) (width 0.25) (layer "B.Cu") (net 16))
 (segment (start 27.94 45.72) (end 27.94 38.1) (width 0.25) (layer "F.Cu") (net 5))
 (segment (start 111.76 83.82) (end 109.22 86.36) (width 0.25) (layer "F.Cu") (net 5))
 (segment (start 27.94 20.32) (end 27.94 35.56) (width 0.25) (layer "F.Cu") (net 5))
 (segment (start 106.68 78.74) (end 111.76 83.82) (width 0.25) (layer "F.Cu") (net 5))
 (segment (start 109.22 86.36) (end 99.06 86.36) (width 0.25) (layer "F.Cu") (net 5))
 (segment (start 27.94 35.56) (end 27.94 38.1) (width 0.25) (layer "F.Cu") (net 5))
 (segment (start 104.26 78.74) (end 106.68 78.74) (width 0.25) (layer "F.Cu") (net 5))
 (segment (start 30.48 45.72) (end 27.94 45.72) (width 0.25) (layer "F.Cu") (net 5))
 (segment (start 99.06 86.36) (end 99.06 88.9) (width 0.25) (layer "F.Cu") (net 5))
 (segment (start 99.06 88.9) (end 86.36 88.9) (width 0.25) (layer "F.Cu") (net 5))
 (via (at 27.94 20.32) (size 0.8) (drill 0.4) (layers "F.Cu" "B.Cu") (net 5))
 (segment (start 27.94 19.3) (end 27.94 20.32) (width 0.25) (layer "B.Cu") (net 5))
 (segment (start 26.42 17.78) (end 27.94 19.3) (width 0.25) (layer "B.Cu") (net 5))
 (segment (start 48.26 43.18) (end 33.02 43.18) (width 0.25) (layer "F.Cu") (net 9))
 (segment (start 33.02 43.18) (end 33.02 38.1) (width 0.25) (layer "F.Cu") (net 9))
 (segment (start 48.26 20.32) (end 48.26 43.18) (width 0.25) (layer "F.Cu") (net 9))
 (via (at 48.26 20.32) (size 0.8) (drill 0.4) (layers "F.Cu" "B.Cu") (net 9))
 (segment (start 48.26 17.78) (end 48.26 20.32) (width 0.25) (layer "B.Cu") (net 9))
 (segment (start 45.72 20.32) (end 45.72 22.86) (width 0.25) (layer "F.Cu") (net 8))
 (segment (start 45.72 40.64) (end 45.72 22.86) (width 0.25) (layer "F.Cu") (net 8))
 (segment (start 35.56 40.64) (end 35.56 38.1) (width 0.25) (layer "F.Cu") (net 8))
 (segment (start 35.56 40.64) (end 45.72 40.64) (width 0.25) (layer "F.Cu") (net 8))
 (via (at 45.72 20.32) (size 0.8) (drill 0.4) (layers "F.Cu" "B.Cu") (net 8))
 (segment (start 45.72 17.78) (end 45.72 20.32) (width 0.25) (layer "B.Cu") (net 8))
 (segment (start 43.18 38.1) (end 38.1 38.1) (width 0.25) (layer "F.Cu") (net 7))
 (segment (start 38.1 45.72) (end 43.18 45.72) (width 0.25) (layer "F.Cu") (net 7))
 (segment (start 43.18 20.32) (end 43.18 38.1) (width 0.25) (layer "F.Cu") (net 7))
 (via (at 43.18 38.1) (size 0.8) (drill 0.4) (layers "F.Cu" "B.Cu") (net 7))
 (via (at 43.18 20.32) (size 0.8) (drill 0.4) (layers "F.Cu" "B.Cu") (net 7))
 (via (at 43.18 45.72) (size 0.8) (drill 0.4) (layers "F.Cu" "B.Cu") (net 7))
 (segment (start 43.18 45.72) (end 43.18 38.1) (width 0.25) (layer "B.Cu") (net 7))
 (segment (start 43.18 19.3) (end 43.18 20.32) (width 0.25) (layer "B.Cu") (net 7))
 (segment (start 41.66 17.78) (end 43.18 19.3) (width 0.25) (layer "B.Cu") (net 7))
 (segment (start 38.1 35.56) (end 40.64 35.56) (width 0.25) (layer "F.Cu") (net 1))
 (segment (start 40.64 20.32) (end 40.64 22.86) (width 0.25) (layer "F.Cu") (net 1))
 (segment (start 40.64 27.94) (end 40.64 35.56) (width 0.25) (layer "F.Cu") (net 1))
 (segment (start 40.64 22.86) (end 40.64 27.94) (width 0.25) (layer "F.Cu") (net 1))
 (via (at 40.64 20.32) (size 0.8) (drill 0.4) (layers "F.Cu" "B.Cu") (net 1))
 (segment (start 39.12 17.78) (end 40.64 19.3) (width 0.25) (layer "B.Cu") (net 1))
 (segment (start 40.64 19.3) (end 40.64 20.32) (width 0.25) (layer "B.Cu") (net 1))
 (via (at 38.1 20.32) (size 0.8) (drill 0.4) (layers "F.Cu" "B.Cu") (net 48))
 (segment (start 38.1 19.3) (end 38.1 20.32) (width 0.25) (layer "B.Cu") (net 48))
 (segment (start 36.58 17.78) (end 38.1 19.3) (width 0.25) (layer "B.Cu") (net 48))
 (segment (start 35.56 35.56) (end 35.56 20.32) (width 0.25) (layer "F.Cu") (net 2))
 (via (at 35.56 20.32) (size 0.8) (drill 0.4) (layers "F.Cu" "B.Cu") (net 2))
 (segment (start 35.56 19.3) (end 35.56 20.32) (width 0.25) (layer "B.Cu") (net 2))
 (segment (start 34.04 17.78) (end 35.56 19.3) (width 0.25) (layer "B.Cu") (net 2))
 (via (at 33.02 20.32) (size 0.8) (drill 0.4) (layers "F.Cu" "B.Cu") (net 49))
 (segment (start 31.5 17.78) (end 33.02 19.3) (width 0.25) (layer "B.Cu") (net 49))
 (segment (start 33.02 19.3) (end 33.02 20.32) (width 0.25) (layer "B.Cu") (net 49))
 (segment (start 33.02 30.48) (end 33.02 35.56) (width 0.25) (layer "F.Cu") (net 3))
 (segment (start 30.48 30.48) (end 33.02 30.48) (width 0.25) (layer "F.Cu") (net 3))
 (segment (start 30.48 20.32) (end 30.48 30.48) (width 0.25) (layer "F.Cu") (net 3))
 (via (at 30.48 20.32) (size 0.8) (drill 0.4) (layers "F.Cu" "B.Cu") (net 3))
 (segment (start 30.48 19.3) (end 30.48 20.32) (width 0.25) (layer "B.Cu") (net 3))
 (segment (start 28.96 17.78) (end 30.48 19.3) (width 0.25) (layer "B.Cu") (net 3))
 (via (at 25.4 20.32) (size 0.8) (drill 0.4) (layers "F.Cu" "B.Cu") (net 50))
 (segment (start 25.4 19.3) (end 25.4 20.32) (width 0.25) (layer "B.Cu") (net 50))
 (segment (start 23.88 17.78) (end 25.4 19.3) (width 0.25) (layer "B.Cu") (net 50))
 (via (at 22.86 20.32) (size 0.8) (drill 0.4) (layers "F.Cu" "B.Cu") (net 51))
 (segment (start 21.34 17.78) (end 22.86 19.3) (width 0.25) (layer "B.Cu") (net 51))
 (segment (start 22.86 19.3) (end 22.86 20.32) (width 0.25) (layer "B.Cu") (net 51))
 (via (at 20.32 20.32) (size 0.8) (drill 0.4) (layers "F.Cu" "B.Cu") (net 52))
 (segment (start 20.32 19.3) (end 20.32 20.32) (width 0.25) (layer "B.Cu") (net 52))
 (segment (start 18.8 17.78) (end 20.32 19.3) (width 0.25) (layer "B.Cu") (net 52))
 (segment (start 99.06 78.74) (end 99.06 81.36) (width 0.25) (layer "F.Cu") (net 21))
 (segment (start 106.88 81.36) (end 109.26 83.74) (width 0.25) (layer "F.Cu") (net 21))
 (segment (start 99.06 81.36) (end 106.88 81.36) (width 0.25) (layer "F.Cu") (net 21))
 (segment (start 30.48 53.88) (end 25.94 53.88) (width 0.25) (layer "F.Cu") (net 6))
 (segment (start 25.4 35.56) (end 25.4 38.1) (width 0.25) (layer "F.Cu") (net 6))
 (segment (start 25.4 38.1) (end 25.4 53.34) (width 0.25) (layer "F.Cu") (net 6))
 (segment (start 25.94 53.88) (end 25.4 53.34) (width 0.25) (layer "F.Cu") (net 6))
 (segment (start 86.36 78.74) (end 91.44 78.74) (width 0.25) (layer "F.Cu") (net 22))
 (segment (start 86.36 29.9) (end 86.36 45.72) (width 0.25) (layer "F.Cu") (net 11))
 (segment (start 119.38 29.9) (end 86.36 29.9) (width 0.25) (layer "F.Cu") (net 11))
 (segment (start 79.86 45.72) (end 86.36 45.72) (width 0.25) (layer "F.Cu") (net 11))
 (segment (start 119.38 34.98) (end 119.38 29.9) (width 0.25) (layer "F.Cu") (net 11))
 (segment (start 116.84 32.44) (end 99.06 32.44) (width 0.25) (layer "F.Cu") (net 33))
 (segment (start 90.8025 37.075) (end 97.3025 37.075) (width 0.25) (layer "F.Cu") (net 33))
 (segment (start 99.06 32.44) (end 97.3025 34.1975) (width 0.25) (layer "F.Cu") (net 33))
 (segment (start 116.84 34.98) (end 116.84 32.44) (width 0.25) (layer "F.Cu") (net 33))
 (segment (start 97.3025 34.1975) (end 97.3025 37.075) (width 0.25) (layer "F.Cu") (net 33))
 (segment (start 114.3 34.98) (end 107.39 41.89) (width 0.25) (layer "F.Cu") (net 36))
 (segment (start 107.39 41.89) (end 107.39 45.72) (width 0.25) (layer "F.Cu") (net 36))
 (segment (start 100.89 45.72) (end 107.39 45.72) (width 0.25) (layer "F.Cu") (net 36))
 (segment (start 97.3025 41.575) (end 90.8025 41.575) (width 0.25) (layer "F.Cu") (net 12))
 (segment (start 137.16 50.22) (end 143.66 50.22) (width 0.25) (layer "F.Cu") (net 12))
 (segment (start 86.36 50.22) (end 79.86 50.22) (width 0.25) (layer "F.Cu") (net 12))
 (segment (start 90.8025 41.575) (end 90.8025 45.7775) (width 0.25) (layer "F.Cu") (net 12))
 (segment (start 86.36 54.695) (end 90.73 59.065) (width 0.25) (layer "F.Cu") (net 12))
 (segment (start 97.3025 41.575) (end 97.3025 46.6325) (width 0.25) (layer "F.Cu") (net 12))
 (segment (start 115.615 59.065) (end 124.46 50.22) (width 0.25) (layer "F.Cu") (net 12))
 (segment (start 97.23 59.065) (end 90.73 59.065) (width 0.25) (layer "F.Cu") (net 12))
 (segment (start 97.3025 46.6325) (end 100.89 50.22) (width 0.25) (layer "F.Cu") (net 12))
 (segment (start 100.085 41.575) (end 97.3025 41.575) (width 0.25) (layer "F.Cu") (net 12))
 (segment (start 101.6 40.06) (end 100.085 41.575) (width 0.25) (layer "F.Cu") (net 12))
 (segment (start 86.36 50.22) (end 86.36 54.695) (width 0.25) (layer "F.Cu") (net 12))
 (segment (start 111.76 34.98) (end 101.6 34.98) (width 0.25) (layer "F.Cu") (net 12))
 (segment (start 97.23 59.065) (end 115.615 59.065) (width 0.25) (layer "F.Cu") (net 12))
 (segment (start 130.96 50.22) (end 137.16 50.22) (width 0.25) (layer "F.Cu") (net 12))
 (segment (start 101.6 34.98) (end 101.6 40.06) (width 0.25) (layer "F.Cu") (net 12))
 (segment (start 124.46 50.22) (end 130.96 50.22) (width 0.25) (layer "F.Cu") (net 12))
 (segment (start 90.8025 45.7775) (end 86.36 50.22) (width 0.25) (layer "F.Cu") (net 12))
 (segment (start 100.89 50.22) (end 107.39 50.22) (width 0.25) (layer "F.Cu") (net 12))
 (segment (start 137.16 37.52) (end 137.16 45.72) (width 0.25) (layer "F.Cu") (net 20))
 (segment (start 137.16 45.72) (end 143.66 45.72) (width 0.25) (layer "F.Cu") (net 20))
 (segment (start 119.38 37.52) (end 137.16 37.52) (width 0.25) (layer "F.Cu") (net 20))
 (segment (start 130.96 45.72) (end 124.46 45.72) (width 0.25) (layer "F.Cu") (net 34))
 (segment (start 116.84 45.14) (end 117.42 45.72) (width 0.25) (layer "F.Cu") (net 34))
 (segment (start 116.84 37.52) (end 116.84 45.14) (width 0.25) (layer "F.Cu") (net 34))
 (segment (start 117.42 45.72) (end 124.46 45.72) (width 0.25) (layer "F.Cu") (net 34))
 (segment (start 112.495 54.565) (end 97.23 54.565) (width 0.25) (layer "F.Cu") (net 32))
 (segment (start 97.23 54.565) (end 90.73 54.565) (width 0.25) (layer "F.Cu") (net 32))
 (segment (start 114.3 52.76) (end 112.495 54.565) (width 0.25) (layer "F.Cu") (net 32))
 (segment (start 114.3 37.52) (end 114.3 52.76) (width 0.25) (layer "F.Cu") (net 32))
 (segment (start 60.96 20.32) (end 60.96 22.86) (width 0.25) (layer "F.Cu") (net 41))
 (segment (start 58.42 27.94) (end 60.96 27.94) (width 0.25) (layer "F.Cu") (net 41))
 (segment (start 60.96 22.86) (end 60.96 27.94) (width 0.25) (layer "F.Cu") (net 41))
 (via (at 60.96 20.32) (size 0.8) (drill 0.4) (layers "F.Cu" "B.Cu") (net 41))
 (segment (start 60.96 17.78) (end 60.96 20.32) (width 0.25) (layer "B.Cu") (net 41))
 (segment (start 58.42 22.86) (end 58.42 25.4) (width 0.25) (layer "F.Cu") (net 40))
 (segment (start 58.42 20.32) (end 58.42 22.86) (width 0.25) (layer "F.Cu") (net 40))
 (via (at 58.42 20.32) (size 0.8) (drill 0.4) (layers "F.Cu" "B.Cu") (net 40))
 (segment (start 58.42 17.78) (end 58.42 20.32) (width 0.25) (layer "B.Cu") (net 40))
 (segment (start 50.8 30.48) (end 50.8 20.32) (width 0.25) (layer "F.Cu") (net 39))
 (segment (start 55.88 30.48) (end 50.8 30.48) (width 0.25) (layer "F.Cu") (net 39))
 (via (at 50.8 20.32) (size 0.8) (drill 0.4) (layers "F.Cu" "B.Cu") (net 39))
 (segment (start 50.8 17.78) (end 50.8 20.32) (width 0.25) (layer "B.Cu") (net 39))
 (segment (start 55.88 25.4) (end 55.88 20.32) (width 0.25) (layer "F.Cu") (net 37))
 (via (at 55.88 20.32) (size 0.8) (drill 0.4) (layers "F.Cu" "B.Cu") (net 37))
 (segment (start 55.88 17.78) (end 55.88 20.32) (width 0.25) (layer "B.Cu") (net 37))
 (segment (start 63.5 20.32) (end 63.5 30.48) (width 0.25) (layer "F.Cu") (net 42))
 (segment (start 63.5 30.48) (end 58.42 30.48) (width 0.25) (layer "F.Cu") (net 42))
 (via (at 63.5 20.32) (size 0.8) (drill 0.4) (layers "F.Cu" "B.Cu") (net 42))
 (segment (start 63.5 17.78) (end 63.5 20.32) (width 0.25) (layer "B.Cu") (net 42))
 (segment (start 53.34 22.86) (end 53.34 27.94) (width 0.25) (layer "F.Cu") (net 38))
 (segment (start 55.88 27.94) (end 53.34 27.94) (width 0.25) (layer "F.Cu") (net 38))
 (segment (start 53.34 22.86) (end 53.34 20.32) (width 0.25) (layer "F.Cu") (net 38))
 (via (at 53.34 20.32) (size 0.8) (drill 0.4) (layers "F.Cu" "B.Cu") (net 38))
 (segment (start 53.34 17.78) (end 53.34 20.32) (width 0.25) (layer "B.Cu") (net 38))
 (segment (start 60.96 55.88) (end 60.96 63.5) (width 0.25) (layer "F.Cu") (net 14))
 (segment (start 58.42 55.88) (end 60.96 55.88) (width 0.25) (layer "F.Cu") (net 14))
 (via (at 60.96 63.5) (size 0.8) (drill 0.4) (layers "F.Cu" "B.Cu") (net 14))
 (segment (start 60.96 66.04) (end 60.96 63.5) (width 0.25) (layer "B.Cu") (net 14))
 (segment (start 55.88 53.34) (end 50.8 53.34) (width 0.25) (layer "F.Cu") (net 19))
 (segment (start 50.8 53.34) (end 50.8 63.5) (width 0.25) (layer "F.Cu") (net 19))
 (via (at 50.8 63.5) (size 0.8) (drill 0.4) (layers "F.Cu" "B.Cu") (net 19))
 (segment (start 50.8 66.04) (end 50.8 63.5) (width 0.25) (layer "B.Cu") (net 19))
 (segment (start 58.42 58.42) (end 58.42 63.5) (width 0.25) (layer "F.Cu") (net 13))
 (via (at 58.42 63.5) (size 0.8) (drill 0.4) (layers "F.Cu" "B.Cu") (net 13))
 (segment (start 58.42 66.04) (end 58.42 63.5) (width 0.25) (layer "B.Cu") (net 13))
 (segment (start 58.42 53.34) (end 63.5 53.34) (width 0.25) (layer "F.Cu") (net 15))
 (segment (start 63.5 53.34) (end 63.5 63.5) (width 0.25) (layer "F.Cu") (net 15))
 (via (at 63.5 63.5) (size 0.8) (drill 0.4) (layers "F.Cu" "B.Cu") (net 15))
 (segment (start 63.5 66.04) (end 63.5 63.5) (width 0.25) (layer "B.Cu") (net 15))
 (segment (start 55.88 60.96) (end 55.88 63.5) (width 0.25) (layer "F.Cu") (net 17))
 (segment (start 55.88 60.96) (end 55.88 58.42) (width 0.25) (layer "F.Cu") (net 17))
 (via (at 55.88 63.5) (size 0.8) (drill 0.4) (layers "F.Cu" "B.Cu") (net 17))
 (segment (start 55.88 66.04) (end 55.88 63.5) (width 0.25) (layer "B.Cu") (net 17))
 (segment (start 53.34 55.88) (end 53.34 63.5) (width 0.25) (layer "F.Cu") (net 18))
 (segment (start 55.88 55.88) (end 53.34 55.88) (width 0.25) (layer "F.Cu") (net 18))
 (via (at 53.34 63.5) (size 0.8) (drill 0.4) (layers "F.Cu" "B.Cu") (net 18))
 (segment (start 53.34 66.04) (end 53.34 63.5) (width 0.25) (layer "B.Cu") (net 18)))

